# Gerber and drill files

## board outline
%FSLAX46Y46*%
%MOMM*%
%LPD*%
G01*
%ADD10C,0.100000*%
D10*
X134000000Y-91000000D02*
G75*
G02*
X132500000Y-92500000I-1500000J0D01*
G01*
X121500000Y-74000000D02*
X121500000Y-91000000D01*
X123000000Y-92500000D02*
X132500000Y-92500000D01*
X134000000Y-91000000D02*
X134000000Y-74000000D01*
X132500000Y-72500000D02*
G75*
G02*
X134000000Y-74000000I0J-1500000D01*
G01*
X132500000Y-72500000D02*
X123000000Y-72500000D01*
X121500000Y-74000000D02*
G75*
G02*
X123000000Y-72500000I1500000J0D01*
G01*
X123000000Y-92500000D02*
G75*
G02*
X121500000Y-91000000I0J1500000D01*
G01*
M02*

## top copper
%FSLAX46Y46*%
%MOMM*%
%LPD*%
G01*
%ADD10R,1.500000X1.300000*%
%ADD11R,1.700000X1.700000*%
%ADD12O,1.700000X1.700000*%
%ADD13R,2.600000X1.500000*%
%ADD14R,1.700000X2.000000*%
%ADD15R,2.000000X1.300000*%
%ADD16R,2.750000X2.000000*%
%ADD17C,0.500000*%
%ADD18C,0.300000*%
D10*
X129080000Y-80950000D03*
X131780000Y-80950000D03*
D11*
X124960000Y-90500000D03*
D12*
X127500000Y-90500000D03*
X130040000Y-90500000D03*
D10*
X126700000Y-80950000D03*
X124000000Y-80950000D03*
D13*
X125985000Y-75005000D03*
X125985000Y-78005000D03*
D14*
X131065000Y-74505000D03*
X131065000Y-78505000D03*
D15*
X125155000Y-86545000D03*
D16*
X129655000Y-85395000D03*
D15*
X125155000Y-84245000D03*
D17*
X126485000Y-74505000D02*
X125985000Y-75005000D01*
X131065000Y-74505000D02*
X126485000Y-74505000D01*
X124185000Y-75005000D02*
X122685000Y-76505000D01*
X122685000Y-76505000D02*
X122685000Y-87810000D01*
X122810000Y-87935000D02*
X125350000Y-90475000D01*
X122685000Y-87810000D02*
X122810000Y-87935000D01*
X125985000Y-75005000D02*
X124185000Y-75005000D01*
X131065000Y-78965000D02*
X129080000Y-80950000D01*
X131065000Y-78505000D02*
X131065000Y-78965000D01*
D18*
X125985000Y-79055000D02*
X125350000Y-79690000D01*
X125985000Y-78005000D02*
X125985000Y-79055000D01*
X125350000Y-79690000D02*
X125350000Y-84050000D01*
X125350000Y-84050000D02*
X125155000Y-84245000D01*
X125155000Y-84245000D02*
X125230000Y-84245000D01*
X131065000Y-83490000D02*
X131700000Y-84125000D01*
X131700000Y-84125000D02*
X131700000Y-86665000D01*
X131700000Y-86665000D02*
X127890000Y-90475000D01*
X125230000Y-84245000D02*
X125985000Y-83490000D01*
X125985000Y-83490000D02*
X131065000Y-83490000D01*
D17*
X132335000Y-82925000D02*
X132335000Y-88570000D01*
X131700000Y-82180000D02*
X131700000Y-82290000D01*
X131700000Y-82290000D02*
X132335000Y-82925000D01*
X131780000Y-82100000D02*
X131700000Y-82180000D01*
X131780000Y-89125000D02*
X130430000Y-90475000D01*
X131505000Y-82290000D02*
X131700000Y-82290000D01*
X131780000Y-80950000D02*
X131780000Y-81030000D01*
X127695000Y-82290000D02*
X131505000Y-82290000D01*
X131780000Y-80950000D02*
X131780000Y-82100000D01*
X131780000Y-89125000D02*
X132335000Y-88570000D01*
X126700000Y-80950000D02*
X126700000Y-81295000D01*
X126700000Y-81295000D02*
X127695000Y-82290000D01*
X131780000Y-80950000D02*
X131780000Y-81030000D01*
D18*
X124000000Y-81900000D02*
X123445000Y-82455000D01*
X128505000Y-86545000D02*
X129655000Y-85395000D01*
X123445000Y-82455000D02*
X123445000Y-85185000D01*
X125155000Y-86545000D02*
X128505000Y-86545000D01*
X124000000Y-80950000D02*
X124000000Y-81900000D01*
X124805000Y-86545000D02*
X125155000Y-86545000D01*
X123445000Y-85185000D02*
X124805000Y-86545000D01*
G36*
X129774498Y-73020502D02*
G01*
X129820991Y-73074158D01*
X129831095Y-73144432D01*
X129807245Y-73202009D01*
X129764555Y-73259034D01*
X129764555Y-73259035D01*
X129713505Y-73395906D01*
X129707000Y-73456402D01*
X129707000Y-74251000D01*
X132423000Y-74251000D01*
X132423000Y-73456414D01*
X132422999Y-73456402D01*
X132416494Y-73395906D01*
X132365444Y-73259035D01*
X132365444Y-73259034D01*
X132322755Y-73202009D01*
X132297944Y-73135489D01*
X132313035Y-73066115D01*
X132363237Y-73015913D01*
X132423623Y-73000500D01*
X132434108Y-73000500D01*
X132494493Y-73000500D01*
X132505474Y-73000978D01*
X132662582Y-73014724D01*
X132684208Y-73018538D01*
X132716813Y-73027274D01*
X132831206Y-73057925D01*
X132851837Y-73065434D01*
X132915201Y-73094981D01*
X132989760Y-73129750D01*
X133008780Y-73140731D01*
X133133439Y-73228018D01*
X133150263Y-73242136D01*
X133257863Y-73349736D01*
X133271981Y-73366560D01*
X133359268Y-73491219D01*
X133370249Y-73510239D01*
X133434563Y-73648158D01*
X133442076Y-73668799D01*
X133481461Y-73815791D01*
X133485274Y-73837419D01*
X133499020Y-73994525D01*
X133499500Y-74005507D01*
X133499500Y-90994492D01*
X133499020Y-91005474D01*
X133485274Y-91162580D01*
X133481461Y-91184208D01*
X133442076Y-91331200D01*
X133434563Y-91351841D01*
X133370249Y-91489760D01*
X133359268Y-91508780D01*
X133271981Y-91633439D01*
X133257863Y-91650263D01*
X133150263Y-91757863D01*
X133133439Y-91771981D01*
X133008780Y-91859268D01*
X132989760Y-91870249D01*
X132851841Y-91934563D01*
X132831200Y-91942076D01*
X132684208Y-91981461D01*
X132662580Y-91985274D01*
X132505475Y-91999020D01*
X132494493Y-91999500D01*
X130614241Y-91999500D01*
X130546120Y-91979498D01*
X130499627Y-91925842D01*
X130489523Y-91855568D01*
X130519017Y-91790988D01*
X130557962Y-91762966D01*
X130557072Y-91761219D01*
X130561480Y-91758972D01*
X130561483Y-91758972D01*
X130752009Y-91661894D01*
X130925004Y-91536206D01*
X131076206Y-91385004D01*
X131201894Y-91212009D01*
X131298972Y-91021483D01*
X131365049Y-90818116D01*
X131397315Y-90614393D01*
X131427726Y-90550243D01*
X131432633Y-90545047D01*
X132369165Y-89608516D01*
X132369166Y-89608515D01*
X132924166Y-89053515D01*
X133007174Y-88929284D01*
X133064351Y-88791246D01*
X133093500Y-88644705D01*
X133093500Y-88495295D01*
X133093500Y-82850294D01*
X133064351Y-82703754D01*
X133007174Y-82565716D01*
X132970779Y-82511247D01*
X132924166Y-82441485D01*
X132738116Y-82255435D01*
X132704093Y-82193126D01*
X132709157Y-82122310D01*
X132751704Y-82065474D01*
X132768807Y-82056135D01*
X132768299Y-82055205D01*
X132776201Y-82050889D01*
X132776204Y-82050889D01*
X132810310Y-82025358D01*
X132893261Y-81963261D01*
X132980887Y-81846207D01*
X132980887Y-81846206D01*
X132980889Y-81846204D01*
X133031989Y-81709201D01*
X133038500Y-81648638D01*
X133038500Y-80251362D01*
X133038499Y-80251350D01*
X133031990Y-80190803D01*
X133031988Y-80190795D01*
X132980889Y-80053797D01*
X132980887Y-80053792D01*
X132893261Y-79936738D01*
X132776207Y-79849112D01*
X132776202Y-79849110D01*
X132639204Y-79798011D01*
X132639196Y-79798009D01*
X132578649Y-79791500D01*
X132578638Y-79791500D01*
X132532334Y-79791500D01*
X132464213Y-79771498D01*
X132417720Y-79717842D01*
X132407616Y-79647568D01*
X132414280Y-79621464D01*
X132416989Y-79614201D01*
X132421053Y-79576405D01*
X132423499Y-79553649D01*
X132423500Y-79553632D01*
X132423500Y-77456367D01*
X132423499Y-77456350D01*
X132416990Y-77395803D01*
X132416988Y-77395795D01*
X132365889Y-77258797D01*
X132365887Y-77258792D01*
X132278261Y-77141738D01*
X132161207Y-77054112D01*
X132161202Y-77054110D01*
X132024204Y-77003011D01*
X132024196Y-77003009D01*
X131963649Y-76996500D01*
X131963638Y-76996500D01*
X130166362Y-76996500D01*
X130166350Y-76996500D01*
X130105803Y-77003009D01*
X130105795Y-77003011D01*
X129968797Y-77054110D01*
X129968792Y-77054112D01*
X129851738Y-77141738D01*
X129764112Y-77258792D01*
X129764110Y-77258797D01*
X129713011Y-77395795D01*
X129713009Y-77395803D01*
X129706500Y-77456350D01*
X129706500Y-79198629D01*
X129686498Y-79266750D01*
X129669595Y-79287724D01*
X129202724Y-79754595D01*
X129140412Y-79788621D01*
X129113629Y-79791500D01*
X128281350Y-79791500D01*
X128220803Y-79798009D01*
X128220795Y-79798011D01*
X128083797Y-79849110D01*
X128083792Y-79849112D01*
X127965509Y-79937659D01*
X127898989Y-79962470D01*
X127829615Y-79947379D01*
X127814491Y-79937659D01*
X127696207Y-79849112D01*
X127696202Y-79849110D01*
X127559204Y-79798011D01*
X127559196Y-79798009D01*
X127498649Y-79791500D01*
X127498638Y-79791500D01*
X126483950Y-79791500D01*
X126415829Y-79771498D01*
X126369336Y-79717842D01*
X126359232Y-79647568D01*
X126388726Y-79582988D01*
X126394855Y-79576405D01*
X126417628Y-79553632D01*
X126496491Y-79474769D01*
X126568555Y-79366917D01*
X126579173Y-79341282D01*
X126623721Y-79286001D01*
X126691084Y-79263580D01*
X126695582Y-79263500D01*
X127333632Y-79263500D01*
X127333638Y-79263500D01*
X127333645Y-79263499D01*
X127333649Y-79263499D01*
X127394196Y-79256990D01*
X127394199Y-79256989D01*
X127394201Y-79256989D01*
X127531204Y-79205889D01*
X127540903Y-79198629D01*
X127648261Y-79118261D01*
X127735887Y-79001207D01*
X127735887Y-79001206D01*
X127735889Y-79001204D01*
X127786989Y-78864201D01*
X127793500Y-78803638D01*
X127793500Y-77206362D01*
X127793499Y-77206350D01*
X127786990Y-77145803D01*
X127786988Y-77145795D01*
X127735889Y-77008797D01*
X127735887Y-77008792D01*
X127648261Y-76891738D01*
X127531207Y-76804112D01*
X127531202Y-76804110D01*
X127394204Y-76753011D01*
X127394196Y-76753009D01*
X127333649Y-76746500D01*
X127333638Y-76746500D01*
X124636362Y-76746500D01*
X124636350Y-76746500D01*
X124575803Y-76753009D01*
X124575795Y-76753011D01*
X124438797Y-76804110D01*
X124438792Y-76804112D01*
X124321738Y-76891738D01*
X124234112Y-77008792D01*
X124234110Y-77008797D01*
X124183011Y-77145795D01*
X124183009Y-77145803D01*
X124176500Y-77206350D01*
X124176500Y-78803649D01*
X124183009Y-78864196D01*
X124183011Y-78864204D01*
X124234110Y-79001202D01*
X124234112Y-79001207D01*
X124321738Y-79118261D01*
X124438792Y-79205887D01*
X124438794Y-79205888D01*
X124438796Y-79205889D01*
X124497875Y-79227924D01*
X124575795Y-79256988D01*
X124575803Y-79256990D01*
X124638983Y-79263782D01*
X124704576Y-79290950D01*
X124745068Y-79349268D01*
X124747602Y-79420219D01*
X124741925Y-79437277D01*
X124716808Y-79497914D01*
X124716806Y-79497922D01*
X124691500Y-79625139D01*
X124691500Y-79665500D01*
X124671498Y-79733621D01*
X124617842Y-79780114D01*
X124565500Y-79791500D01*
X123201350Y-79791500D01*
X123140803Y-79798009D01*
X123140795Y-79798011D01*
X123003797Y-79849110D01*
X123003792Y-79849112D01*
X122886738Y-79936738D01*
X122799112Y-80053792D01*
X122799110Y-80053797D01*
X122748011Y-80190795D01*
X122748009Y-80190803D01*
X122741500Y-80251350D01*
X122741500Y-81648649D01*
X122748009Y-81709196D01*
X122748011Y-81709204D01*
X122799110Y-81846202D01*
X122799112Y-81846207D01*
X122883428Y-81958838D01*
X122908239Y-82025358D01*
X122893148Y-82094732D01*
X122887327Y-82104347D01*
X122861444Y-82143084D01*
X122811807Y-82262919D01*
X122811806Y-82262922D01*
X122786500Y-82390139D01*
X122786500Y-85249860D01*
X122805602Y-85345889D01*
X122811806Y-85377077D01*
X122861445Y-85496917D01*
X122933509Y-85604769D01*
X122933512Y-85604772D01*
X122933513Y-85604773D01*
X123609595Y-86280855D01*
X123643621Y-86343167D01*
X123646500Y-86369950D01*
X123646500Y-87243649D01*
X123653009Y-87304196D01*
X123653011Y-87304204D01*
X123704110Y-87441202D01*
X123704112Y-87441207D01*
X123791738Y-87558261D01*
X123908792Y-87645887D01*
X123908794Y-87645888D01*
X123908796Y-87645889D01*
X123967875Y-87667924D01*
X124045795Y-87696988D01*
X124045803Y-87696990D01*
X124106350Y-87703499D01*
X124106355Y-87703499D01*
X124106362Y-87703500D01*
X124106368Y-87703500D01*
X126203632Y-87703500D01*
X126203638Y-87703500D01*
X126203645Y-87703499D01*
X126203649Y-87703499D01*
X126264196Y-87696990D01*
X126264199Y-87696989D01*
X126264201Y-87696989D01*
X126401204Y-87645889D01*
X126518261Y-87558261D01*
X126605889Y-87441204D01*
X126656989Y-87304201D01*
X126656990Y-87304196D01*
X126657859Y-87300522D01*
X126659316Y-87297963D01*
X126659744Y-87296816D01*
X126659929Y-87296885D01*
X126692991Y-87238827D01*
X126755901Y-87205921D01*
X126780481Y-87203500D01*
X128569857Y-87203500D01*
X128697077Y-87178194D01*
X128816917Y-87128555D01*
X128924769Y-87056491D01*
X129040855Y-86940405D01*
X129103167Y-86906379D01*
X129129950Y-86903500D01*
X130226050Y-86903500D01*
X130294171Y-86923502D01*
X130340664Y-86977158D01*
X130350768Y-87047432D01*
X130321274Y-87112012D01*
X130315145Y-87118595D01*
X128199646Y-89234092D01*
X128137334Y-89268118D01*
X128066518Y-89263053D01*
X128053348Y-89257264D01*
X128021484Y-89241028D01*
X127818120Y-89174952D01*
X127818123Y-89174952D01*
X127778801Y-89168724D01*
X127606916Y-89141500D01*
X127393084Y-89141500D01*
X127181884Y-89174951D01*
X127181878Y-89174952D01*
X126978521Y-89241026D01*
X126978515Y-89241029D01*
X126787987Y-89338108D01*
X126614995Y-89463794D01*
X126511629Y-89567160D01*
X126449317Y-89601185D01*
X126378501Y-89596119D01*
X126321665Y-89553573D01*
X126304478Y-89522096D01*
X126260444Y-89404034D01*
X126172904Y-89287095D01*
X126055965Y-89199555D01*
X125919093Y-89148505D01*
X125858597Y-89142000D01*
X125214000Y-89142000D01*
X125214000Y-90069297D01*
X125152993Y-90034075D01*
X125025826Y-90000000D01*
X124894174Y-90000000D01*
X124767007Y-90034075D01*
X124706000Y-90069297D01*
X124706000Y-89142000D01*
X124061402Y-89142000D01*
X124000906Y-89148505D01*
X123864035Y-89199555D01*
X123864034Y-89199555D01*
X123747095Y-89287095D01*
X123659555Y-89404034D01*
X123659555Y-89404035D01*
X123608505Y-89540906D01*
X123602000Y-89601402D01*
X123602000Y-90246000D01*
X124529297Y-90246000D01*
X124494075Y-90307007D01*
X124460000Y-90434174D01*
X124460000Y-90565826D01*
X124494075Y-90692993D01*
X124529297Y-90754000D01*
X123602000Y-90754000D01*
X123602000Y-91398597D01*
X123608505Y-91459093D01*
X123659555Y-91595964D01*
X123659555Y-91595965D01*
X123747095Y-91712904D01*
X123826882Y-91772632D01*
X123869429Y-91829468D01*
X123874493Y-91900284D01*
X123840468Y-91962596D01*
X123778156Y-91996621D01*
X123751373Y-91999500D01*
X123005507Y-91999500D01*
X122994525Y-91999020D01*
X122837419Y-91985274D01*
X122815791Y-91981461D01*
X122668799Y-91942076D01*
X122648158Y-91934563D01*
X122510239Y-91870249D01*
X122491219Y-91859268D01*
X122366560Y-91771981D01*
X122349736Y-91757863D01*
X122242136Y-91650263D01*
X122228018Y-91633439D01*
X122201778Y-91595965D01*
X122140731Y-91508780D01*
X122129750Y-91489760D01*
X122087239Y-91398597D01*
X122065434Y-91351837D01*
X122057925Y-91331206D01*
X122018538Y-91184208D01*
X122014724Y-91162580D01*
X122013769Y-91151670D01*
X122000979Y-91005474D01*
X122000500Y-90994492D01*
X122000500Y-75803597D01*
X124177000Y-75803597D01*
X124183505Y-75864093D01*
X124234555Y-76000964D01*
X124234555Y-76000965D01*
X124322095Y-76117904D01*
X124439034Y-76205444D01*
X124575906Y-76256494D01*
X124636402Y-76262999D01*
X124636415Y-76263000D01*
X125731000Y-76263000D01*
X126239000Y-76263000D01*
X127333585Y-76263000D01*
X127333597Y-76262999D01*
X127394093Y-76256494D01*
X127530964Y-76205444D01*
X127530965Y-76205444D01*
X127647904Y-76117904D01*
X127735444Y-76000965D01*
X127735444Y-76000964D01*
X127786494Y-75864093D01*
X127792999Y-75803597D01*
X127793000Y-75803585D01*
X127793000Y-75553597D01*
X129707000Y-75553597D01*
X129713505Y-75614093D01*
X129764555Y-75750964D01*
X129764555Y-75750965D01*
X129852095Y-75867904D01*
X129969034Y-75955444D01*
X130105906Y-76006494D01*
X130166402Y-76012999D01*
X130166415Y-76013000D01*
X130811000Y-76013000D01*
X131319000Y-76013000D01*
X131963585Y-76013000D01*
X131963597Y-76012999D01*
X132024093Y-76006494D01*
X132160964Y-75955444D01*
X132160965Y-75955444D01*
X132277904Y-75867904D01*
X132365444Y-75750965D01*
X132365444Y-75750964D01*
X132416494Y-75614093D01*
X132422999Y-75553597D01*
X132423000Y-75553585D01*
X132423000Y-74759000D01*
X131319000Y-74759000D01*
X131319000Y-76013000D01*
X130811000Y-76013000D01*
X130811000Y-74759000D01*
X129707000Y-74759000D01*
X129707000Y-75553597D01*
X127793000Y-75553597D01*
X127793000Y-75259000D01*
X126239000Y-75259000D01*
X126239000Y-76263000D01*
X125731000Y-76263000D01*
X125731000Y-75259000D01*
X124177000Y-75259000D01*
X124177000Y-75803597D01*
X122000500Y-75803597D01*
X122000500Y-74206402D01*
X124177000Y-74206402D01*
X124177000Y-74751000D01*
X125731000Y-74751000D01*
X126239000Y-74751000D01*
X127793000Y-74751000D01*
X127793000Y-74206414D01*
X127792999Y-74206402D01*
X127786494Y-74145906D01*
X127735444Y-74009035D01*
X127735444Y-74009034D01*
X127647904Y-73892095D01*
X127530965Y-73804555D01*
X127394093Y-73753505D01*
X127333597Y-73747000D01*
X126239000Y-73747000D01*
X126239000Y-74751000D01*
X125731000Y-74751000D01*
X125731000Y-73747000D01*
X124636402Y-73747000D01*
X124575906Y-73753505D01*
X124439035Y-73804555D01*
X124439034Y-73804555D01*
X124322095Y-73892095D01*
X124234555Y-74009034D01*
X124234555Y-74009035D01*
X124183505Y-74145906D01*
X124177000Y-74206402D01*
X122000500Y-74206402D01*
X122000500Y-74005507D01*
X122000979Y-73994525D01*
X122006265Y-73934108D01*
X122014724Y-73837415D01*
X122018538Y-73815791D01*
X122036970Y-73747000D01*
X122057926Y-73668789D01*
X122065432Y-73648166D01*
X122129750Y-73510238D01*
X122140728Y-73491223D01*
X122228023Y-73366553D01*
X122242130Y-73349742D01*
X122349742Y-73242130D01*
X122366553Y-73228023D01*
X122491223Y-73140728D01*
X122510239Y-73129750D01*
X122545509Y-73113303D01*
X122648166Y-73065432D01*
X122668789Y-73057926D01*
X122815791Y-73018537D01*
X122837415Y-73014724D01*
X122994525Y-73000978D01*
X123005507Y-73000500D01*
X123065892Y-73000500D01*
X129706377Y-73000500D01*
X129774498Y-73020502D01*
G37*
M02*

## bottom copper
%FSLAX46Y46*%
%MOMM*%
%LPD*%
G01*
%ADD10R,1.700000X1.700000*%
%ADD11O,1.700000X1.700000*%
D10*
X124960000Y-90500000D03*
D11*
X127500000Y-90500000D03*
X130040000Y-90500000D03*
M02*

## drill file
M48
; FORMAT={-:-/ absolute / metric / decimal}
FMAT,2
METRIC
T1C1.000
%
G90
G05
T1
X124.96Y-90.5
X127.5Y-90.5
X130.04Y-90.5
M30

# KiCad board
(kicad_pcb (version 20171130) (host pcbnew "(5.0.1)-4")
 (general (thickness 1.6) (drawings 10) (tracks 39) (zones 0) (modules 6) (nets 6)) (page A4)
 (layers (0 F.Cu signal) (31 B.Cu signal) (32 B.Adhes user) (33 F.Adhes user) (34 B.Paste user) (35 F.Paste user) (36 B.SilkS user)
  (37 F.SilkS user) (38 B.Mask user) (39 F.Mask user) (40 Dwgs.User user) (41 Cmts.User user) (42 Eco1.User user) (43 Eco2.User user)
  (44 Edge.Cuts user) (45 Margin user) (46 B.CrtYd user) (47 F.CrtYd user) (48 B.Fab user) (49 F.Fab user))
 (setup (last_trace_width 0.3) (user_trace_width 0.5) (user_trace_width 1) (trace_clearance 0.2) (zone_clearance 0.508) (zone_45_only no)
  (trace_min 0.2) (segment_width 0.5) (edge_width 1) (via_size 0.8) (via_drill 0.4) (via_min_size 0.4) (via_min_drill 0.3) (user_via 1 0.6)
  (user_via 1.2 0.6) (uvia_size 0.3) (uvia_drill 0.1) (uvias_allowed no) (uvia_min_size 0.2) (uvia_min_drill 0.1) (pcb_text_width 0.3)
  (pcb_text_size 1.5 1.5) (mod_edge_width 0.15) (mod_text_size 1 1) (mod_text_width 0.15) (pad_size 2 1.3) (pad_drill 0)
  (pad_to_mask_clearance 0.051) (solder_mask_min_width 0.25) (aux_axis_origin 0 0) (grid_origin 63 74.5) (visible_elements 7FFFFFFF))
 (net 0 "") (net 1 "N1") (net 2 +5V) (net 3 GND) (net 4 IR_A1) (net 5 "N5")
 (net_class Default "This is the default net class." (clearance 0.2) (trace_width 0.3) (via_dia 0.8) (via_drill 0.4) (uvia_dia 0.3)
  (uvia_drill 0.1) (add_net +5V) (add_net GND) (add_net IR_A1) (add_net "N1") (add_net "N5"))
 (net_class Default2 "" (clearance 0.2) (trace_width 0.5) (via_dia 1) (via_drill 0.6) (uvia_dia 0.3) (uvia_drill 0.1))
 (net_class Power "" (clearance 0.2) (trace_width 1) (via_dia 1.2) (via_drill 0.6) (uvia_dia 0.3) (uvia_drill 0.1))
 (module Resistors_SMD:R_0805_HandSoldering (layer F.Cu) (at 130.43 80.95 180)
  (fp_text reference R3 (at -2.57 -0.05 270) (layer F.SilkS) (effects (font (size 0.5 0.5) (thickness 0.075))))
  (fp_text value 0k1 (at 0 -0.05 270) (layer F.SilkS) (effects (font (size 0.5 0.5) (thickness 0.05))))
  (pad 2 smd rect (at 1.35 0 180) (size 1.5 1.3) (layers F.Cu F.Paste F.Mask) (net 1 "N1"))
  (pad 1 smd rect (at -1.35 0 180) (size 1.5 1.3) (layers F.Cu F.Paste F.Mask) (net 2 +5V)))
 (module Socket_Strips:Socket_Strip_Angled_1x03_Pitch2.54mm (layer F.Cu) (at 124.96 90.5 90)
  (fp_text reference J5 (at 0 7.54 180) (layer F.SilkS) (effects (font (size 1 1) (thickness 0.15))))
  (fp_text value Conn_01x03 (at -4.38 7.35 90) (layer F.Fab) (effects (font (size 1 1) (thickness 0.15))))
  (pad 1 thru_hole rect (at 0 0 90) (size 1.7 1.7) (drill 1) (layers *.Cu *.Mask) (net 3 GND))
  (pad 2 thru_hole oval (at 0 2.54 90) (size 1.7 1.7) (drill 1) (layers *.Cu *.Mask) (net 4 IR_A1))
  (pad 3 thru_hole oval (at 0 5.08 90) (size 1.7 1.7) (drill 1) (layers *.Cu *.Mask) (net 2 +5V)))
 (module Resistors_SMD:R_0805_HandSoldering (layer F.Cu) (at 125.35 80.95 180)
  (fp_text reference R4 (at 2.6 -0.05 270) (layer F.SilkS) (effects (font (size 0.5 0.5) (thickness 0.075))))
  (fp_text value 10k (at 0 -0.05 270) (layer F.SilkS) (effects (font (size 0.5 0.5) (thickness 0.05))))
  (pad 1 smd rect (at -1.35 0 180) (size 1.5 1.3) (layers F.Cu F.Paste F.Mask) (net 2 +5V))
  (pad 2 smd rect (at 1.35 0 180) (size 1.5 1.3) (layers F.Cu F.Paste F.Mask) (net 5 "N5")))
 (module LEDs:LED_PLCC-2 (layer F.Cu) (at 125.985 76.505 270)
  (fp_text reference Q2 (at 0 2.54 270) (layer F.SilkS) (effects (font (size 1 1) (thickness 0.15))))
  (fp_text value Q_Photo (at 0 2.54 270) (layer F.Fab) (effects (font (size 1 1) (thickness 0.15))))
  (pad 1 smd rect (at -1.5 0 270) (size 1.5 2.6) (layers F.Cu F.Paste F.Mask) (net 3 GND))
  (pad 2 smd rect (at 1.5 0 270) (size 1.5 2.6) (layers F.Cu F.Paste F.Mask) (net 4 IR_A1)))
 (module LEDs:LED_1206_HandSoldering (layer F.Cu) (at 131.065 76.505 270)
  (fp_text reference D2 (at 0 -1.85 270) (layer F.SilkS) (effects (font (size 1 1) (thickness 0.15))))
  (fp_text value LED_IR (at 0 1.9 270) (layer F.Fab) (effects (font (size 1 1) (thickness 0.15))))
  (pad 1 smd rect (at -2 0 270) (size 2 1.7) (layers F.Cu F.Paste F.Mask) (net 3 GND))
  (pad 2 smd rect (at 2 0 270) (size 2 1.7) (layers F.Cu F.Paste F.Mask) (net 1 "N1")))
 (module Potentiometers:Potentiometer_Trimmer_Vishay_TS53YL (layer F.Cu) (at 127.255 85.395 180)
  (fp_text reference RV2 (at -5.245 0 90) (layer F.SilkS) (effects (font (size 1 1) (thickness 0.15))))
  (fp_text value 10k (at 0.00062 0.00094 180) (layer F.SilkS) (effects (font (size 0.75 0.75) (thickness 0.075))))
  (pad 1 smd rect (at 2.1 -1.15 180) (size 2 1.3) (layers F.Cu F.Mask) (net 5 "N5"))
  (pad 2 smd rect (at -2.4 0 180) (size 2.75 2) (layers F.Cu F.Mask) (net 5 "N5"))
  (pad 3 smd rect (at 2.1 1.15 180) (size 2 1.3) (layers F.Cu F.Mask) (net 4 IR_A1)))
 (gr_arc (start 132.5 91) (end 132.5 92.5) (angle -90) (layer Edge.Cuts) (width 0.1))
 (gr_line (start 121.5 74) (end 121.5 91) (layer Edge.Cuts) (width 0.1))
 (gr_line (start 123 92.5) (end 132.5 92.5) (layer Edge.Cuts) (width 0.1))
 (gr_line (start 134 91) (end 134 74) (layer Edge.Cuts) (width 0.1))
 (gr_arc (start 132.5 74) (end 134 74) (angle -90) (layer Edge.Cuts) (width 0.1))
 (gr_line (start 132.5 72.5) (end 123 72.5) (layer Edge.Cuts) (width 0.1))
 (gr_arc (start 123 74) (end 123 72.5) (angle -90) (layer Edge.Cuts) (width 0.1))
 (gr_arc (start 123 91) (end 121.5 91) (angle -90) (layer Edge.Cuts) (width 0.1))
 (segment (start 126.485 74.505) (end 125.985 75.005) (width 0.5) (layer F.Cu) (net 3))
 (segment (start 131.065 74.505) (end 126.485 74.505) (width 0.5) (layer F.Cu) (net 3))
 (segment (start 124.185 75.005) (end 122.685 76.505) (width 0.5) (layer F.Cu) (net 3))
 (segment (start 122.685 76.505) (end 122.685 87.81) (width 0.5) (layer F.Cu) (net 3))
 (segment (start 122.81 87.935) (end 125.35 90.475) (width 0.5) (layer F.Cu) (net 3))
 (segment (start 122.685 87.81) (end 122.81 87.935) (width 0.5) (layer F.Cu) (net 3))
 (segment (start 125.985 75.005) (end 124.185 75.005) (width 0.5) (layer F.Cu) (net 3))
 (segment (start 131.065 78.965) (end 129.08 80.95) (width 0.5) (layer F.Cu) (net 1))
 (segment (start 131.065 78.505) (end 131.065 78.965) (width 0.5) (layer F.Cu) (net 1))
 (segment (start 125.985 79.055) (end 125.35 79.69) (width 0.3) (layer F.Cu) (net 4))
 (segment (start 125.985 78.005) (end 125.985 79.055) (width 0.3) (layer F.Cu) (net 4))
 (segment (start 125.35 79.69) (end 125.35 84.05) (width 0.3) (layer F.Cu) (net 4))
 (segment (start 125.35 84.05) (end 125.155 84.245) (width 0.3) (layer F.Cu) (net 4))
 (segment (start 125.155 84.245) (end 125.23 84.245) (width 0.3) (layer F.Cu) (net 4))
 (segment (start 131.065 83.49) (end 131.7 84.125) (width 0.3) (layer F.Cu) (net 4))
 (segment (start 131.7 84.125) (end 131.7 86.665) (width 0.3) (layer F.Cu) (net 4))
 (segment (start 131.7 86.665) (end 127.89 90.475) (width 0.3) (layer F.Cu) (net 4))
 (segment (start 125.23 84.245) (end 125.985 83.49) (width 0.3) (layer F.Cu) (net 4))
 (segment (start 125.985 83.49) (end 131.065 83.49) (width 0.3) (layer F.Cu) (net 4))
 (segment (start 132.335 82.925) (end 132.335 88.57) (width 0.5) (layer F.Cu) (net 2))
 (segment (start 131.7 82.18) (end 131.7 82.29) (width 0.5) (layer F.Cu) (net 2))
 (segment (start 131.7 82.29) (end 132.335 82.925) (width 0.5) (layer F.Cu) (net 2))
 (segment (start 131.78 82.1) (end 131.7 82.18) (width 0.5) (layer F.Cu) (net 2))
 (segment (start 131.78 89.125) (end 130.43 90.475) (width 0.5) (layer F.Cu) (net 2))
 (segment (start 131.505 82.29) (end 131.7 82.29) (width 0.5) (layer F.Cu) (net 2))
 (segment (start 131.78 80.95) (end 131.78 81.03) (width 0.5) (layer F.Cu) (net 2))
 (segment (start 127.695 82.29) (end 131.505 82.29) (width 0.5) (layer F.Cu) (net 2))
 (segment (start 131.78 80.95) (end 131.78 82.1) (width 0.5) (layer F.Cu) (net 2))
 (segment (start 131.78 89.125) (end 132.335 88.57) (width 0.5) (layer F.Cu) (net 2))
 (segment (start 126.7 80.95) (end 126.7 81.295) (width 0.5) (layer F.Cu) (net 2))
 (segment (start 126.7 81.295) (end 127.695 82.29) (width 0.5) (layer F.Cu) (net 2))
 (segment (start 131.78 80.95) (end 131.78 81.03) (width 0.5) (layer F.Cu) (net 2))
 (segment (start 124 81.9) (end 123.445 82.455) (width 0.3) (layer F.Cu) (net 5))
 (segment (start 128.505 86.545) (end 129.655 85.395) (width 0.3) (layer F.Cu) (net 5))
 (segment (start 123.445 82.455) (end 123.445 85.185) (width 0.3) (layer F.Cu) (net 5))
 (segment (start 125.155 86.545) (end 128.505 86.545) (width 0.3) (layer F.Cu) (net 5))
 (segment (start 124 80.95) (end 124 81.9) (width 0.3) (layer F.Cu) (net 5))
 (segment (start 124.805 86.545) (end 125.155 86.545) (width 0.3) (layer F.Cu) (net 5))
 (segment (start 123.445 85.185) (end 124.805 86.545) (width 0.3) (layer F.Cu) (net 5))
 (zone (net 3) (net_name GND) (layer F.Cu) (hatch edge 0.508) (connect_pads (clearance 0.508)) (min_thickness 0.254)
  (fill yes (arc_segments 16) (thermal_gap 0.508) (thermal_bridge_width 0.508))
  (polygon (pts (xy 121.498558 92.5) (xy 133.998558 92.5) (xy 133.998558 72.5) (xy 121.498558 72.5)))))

